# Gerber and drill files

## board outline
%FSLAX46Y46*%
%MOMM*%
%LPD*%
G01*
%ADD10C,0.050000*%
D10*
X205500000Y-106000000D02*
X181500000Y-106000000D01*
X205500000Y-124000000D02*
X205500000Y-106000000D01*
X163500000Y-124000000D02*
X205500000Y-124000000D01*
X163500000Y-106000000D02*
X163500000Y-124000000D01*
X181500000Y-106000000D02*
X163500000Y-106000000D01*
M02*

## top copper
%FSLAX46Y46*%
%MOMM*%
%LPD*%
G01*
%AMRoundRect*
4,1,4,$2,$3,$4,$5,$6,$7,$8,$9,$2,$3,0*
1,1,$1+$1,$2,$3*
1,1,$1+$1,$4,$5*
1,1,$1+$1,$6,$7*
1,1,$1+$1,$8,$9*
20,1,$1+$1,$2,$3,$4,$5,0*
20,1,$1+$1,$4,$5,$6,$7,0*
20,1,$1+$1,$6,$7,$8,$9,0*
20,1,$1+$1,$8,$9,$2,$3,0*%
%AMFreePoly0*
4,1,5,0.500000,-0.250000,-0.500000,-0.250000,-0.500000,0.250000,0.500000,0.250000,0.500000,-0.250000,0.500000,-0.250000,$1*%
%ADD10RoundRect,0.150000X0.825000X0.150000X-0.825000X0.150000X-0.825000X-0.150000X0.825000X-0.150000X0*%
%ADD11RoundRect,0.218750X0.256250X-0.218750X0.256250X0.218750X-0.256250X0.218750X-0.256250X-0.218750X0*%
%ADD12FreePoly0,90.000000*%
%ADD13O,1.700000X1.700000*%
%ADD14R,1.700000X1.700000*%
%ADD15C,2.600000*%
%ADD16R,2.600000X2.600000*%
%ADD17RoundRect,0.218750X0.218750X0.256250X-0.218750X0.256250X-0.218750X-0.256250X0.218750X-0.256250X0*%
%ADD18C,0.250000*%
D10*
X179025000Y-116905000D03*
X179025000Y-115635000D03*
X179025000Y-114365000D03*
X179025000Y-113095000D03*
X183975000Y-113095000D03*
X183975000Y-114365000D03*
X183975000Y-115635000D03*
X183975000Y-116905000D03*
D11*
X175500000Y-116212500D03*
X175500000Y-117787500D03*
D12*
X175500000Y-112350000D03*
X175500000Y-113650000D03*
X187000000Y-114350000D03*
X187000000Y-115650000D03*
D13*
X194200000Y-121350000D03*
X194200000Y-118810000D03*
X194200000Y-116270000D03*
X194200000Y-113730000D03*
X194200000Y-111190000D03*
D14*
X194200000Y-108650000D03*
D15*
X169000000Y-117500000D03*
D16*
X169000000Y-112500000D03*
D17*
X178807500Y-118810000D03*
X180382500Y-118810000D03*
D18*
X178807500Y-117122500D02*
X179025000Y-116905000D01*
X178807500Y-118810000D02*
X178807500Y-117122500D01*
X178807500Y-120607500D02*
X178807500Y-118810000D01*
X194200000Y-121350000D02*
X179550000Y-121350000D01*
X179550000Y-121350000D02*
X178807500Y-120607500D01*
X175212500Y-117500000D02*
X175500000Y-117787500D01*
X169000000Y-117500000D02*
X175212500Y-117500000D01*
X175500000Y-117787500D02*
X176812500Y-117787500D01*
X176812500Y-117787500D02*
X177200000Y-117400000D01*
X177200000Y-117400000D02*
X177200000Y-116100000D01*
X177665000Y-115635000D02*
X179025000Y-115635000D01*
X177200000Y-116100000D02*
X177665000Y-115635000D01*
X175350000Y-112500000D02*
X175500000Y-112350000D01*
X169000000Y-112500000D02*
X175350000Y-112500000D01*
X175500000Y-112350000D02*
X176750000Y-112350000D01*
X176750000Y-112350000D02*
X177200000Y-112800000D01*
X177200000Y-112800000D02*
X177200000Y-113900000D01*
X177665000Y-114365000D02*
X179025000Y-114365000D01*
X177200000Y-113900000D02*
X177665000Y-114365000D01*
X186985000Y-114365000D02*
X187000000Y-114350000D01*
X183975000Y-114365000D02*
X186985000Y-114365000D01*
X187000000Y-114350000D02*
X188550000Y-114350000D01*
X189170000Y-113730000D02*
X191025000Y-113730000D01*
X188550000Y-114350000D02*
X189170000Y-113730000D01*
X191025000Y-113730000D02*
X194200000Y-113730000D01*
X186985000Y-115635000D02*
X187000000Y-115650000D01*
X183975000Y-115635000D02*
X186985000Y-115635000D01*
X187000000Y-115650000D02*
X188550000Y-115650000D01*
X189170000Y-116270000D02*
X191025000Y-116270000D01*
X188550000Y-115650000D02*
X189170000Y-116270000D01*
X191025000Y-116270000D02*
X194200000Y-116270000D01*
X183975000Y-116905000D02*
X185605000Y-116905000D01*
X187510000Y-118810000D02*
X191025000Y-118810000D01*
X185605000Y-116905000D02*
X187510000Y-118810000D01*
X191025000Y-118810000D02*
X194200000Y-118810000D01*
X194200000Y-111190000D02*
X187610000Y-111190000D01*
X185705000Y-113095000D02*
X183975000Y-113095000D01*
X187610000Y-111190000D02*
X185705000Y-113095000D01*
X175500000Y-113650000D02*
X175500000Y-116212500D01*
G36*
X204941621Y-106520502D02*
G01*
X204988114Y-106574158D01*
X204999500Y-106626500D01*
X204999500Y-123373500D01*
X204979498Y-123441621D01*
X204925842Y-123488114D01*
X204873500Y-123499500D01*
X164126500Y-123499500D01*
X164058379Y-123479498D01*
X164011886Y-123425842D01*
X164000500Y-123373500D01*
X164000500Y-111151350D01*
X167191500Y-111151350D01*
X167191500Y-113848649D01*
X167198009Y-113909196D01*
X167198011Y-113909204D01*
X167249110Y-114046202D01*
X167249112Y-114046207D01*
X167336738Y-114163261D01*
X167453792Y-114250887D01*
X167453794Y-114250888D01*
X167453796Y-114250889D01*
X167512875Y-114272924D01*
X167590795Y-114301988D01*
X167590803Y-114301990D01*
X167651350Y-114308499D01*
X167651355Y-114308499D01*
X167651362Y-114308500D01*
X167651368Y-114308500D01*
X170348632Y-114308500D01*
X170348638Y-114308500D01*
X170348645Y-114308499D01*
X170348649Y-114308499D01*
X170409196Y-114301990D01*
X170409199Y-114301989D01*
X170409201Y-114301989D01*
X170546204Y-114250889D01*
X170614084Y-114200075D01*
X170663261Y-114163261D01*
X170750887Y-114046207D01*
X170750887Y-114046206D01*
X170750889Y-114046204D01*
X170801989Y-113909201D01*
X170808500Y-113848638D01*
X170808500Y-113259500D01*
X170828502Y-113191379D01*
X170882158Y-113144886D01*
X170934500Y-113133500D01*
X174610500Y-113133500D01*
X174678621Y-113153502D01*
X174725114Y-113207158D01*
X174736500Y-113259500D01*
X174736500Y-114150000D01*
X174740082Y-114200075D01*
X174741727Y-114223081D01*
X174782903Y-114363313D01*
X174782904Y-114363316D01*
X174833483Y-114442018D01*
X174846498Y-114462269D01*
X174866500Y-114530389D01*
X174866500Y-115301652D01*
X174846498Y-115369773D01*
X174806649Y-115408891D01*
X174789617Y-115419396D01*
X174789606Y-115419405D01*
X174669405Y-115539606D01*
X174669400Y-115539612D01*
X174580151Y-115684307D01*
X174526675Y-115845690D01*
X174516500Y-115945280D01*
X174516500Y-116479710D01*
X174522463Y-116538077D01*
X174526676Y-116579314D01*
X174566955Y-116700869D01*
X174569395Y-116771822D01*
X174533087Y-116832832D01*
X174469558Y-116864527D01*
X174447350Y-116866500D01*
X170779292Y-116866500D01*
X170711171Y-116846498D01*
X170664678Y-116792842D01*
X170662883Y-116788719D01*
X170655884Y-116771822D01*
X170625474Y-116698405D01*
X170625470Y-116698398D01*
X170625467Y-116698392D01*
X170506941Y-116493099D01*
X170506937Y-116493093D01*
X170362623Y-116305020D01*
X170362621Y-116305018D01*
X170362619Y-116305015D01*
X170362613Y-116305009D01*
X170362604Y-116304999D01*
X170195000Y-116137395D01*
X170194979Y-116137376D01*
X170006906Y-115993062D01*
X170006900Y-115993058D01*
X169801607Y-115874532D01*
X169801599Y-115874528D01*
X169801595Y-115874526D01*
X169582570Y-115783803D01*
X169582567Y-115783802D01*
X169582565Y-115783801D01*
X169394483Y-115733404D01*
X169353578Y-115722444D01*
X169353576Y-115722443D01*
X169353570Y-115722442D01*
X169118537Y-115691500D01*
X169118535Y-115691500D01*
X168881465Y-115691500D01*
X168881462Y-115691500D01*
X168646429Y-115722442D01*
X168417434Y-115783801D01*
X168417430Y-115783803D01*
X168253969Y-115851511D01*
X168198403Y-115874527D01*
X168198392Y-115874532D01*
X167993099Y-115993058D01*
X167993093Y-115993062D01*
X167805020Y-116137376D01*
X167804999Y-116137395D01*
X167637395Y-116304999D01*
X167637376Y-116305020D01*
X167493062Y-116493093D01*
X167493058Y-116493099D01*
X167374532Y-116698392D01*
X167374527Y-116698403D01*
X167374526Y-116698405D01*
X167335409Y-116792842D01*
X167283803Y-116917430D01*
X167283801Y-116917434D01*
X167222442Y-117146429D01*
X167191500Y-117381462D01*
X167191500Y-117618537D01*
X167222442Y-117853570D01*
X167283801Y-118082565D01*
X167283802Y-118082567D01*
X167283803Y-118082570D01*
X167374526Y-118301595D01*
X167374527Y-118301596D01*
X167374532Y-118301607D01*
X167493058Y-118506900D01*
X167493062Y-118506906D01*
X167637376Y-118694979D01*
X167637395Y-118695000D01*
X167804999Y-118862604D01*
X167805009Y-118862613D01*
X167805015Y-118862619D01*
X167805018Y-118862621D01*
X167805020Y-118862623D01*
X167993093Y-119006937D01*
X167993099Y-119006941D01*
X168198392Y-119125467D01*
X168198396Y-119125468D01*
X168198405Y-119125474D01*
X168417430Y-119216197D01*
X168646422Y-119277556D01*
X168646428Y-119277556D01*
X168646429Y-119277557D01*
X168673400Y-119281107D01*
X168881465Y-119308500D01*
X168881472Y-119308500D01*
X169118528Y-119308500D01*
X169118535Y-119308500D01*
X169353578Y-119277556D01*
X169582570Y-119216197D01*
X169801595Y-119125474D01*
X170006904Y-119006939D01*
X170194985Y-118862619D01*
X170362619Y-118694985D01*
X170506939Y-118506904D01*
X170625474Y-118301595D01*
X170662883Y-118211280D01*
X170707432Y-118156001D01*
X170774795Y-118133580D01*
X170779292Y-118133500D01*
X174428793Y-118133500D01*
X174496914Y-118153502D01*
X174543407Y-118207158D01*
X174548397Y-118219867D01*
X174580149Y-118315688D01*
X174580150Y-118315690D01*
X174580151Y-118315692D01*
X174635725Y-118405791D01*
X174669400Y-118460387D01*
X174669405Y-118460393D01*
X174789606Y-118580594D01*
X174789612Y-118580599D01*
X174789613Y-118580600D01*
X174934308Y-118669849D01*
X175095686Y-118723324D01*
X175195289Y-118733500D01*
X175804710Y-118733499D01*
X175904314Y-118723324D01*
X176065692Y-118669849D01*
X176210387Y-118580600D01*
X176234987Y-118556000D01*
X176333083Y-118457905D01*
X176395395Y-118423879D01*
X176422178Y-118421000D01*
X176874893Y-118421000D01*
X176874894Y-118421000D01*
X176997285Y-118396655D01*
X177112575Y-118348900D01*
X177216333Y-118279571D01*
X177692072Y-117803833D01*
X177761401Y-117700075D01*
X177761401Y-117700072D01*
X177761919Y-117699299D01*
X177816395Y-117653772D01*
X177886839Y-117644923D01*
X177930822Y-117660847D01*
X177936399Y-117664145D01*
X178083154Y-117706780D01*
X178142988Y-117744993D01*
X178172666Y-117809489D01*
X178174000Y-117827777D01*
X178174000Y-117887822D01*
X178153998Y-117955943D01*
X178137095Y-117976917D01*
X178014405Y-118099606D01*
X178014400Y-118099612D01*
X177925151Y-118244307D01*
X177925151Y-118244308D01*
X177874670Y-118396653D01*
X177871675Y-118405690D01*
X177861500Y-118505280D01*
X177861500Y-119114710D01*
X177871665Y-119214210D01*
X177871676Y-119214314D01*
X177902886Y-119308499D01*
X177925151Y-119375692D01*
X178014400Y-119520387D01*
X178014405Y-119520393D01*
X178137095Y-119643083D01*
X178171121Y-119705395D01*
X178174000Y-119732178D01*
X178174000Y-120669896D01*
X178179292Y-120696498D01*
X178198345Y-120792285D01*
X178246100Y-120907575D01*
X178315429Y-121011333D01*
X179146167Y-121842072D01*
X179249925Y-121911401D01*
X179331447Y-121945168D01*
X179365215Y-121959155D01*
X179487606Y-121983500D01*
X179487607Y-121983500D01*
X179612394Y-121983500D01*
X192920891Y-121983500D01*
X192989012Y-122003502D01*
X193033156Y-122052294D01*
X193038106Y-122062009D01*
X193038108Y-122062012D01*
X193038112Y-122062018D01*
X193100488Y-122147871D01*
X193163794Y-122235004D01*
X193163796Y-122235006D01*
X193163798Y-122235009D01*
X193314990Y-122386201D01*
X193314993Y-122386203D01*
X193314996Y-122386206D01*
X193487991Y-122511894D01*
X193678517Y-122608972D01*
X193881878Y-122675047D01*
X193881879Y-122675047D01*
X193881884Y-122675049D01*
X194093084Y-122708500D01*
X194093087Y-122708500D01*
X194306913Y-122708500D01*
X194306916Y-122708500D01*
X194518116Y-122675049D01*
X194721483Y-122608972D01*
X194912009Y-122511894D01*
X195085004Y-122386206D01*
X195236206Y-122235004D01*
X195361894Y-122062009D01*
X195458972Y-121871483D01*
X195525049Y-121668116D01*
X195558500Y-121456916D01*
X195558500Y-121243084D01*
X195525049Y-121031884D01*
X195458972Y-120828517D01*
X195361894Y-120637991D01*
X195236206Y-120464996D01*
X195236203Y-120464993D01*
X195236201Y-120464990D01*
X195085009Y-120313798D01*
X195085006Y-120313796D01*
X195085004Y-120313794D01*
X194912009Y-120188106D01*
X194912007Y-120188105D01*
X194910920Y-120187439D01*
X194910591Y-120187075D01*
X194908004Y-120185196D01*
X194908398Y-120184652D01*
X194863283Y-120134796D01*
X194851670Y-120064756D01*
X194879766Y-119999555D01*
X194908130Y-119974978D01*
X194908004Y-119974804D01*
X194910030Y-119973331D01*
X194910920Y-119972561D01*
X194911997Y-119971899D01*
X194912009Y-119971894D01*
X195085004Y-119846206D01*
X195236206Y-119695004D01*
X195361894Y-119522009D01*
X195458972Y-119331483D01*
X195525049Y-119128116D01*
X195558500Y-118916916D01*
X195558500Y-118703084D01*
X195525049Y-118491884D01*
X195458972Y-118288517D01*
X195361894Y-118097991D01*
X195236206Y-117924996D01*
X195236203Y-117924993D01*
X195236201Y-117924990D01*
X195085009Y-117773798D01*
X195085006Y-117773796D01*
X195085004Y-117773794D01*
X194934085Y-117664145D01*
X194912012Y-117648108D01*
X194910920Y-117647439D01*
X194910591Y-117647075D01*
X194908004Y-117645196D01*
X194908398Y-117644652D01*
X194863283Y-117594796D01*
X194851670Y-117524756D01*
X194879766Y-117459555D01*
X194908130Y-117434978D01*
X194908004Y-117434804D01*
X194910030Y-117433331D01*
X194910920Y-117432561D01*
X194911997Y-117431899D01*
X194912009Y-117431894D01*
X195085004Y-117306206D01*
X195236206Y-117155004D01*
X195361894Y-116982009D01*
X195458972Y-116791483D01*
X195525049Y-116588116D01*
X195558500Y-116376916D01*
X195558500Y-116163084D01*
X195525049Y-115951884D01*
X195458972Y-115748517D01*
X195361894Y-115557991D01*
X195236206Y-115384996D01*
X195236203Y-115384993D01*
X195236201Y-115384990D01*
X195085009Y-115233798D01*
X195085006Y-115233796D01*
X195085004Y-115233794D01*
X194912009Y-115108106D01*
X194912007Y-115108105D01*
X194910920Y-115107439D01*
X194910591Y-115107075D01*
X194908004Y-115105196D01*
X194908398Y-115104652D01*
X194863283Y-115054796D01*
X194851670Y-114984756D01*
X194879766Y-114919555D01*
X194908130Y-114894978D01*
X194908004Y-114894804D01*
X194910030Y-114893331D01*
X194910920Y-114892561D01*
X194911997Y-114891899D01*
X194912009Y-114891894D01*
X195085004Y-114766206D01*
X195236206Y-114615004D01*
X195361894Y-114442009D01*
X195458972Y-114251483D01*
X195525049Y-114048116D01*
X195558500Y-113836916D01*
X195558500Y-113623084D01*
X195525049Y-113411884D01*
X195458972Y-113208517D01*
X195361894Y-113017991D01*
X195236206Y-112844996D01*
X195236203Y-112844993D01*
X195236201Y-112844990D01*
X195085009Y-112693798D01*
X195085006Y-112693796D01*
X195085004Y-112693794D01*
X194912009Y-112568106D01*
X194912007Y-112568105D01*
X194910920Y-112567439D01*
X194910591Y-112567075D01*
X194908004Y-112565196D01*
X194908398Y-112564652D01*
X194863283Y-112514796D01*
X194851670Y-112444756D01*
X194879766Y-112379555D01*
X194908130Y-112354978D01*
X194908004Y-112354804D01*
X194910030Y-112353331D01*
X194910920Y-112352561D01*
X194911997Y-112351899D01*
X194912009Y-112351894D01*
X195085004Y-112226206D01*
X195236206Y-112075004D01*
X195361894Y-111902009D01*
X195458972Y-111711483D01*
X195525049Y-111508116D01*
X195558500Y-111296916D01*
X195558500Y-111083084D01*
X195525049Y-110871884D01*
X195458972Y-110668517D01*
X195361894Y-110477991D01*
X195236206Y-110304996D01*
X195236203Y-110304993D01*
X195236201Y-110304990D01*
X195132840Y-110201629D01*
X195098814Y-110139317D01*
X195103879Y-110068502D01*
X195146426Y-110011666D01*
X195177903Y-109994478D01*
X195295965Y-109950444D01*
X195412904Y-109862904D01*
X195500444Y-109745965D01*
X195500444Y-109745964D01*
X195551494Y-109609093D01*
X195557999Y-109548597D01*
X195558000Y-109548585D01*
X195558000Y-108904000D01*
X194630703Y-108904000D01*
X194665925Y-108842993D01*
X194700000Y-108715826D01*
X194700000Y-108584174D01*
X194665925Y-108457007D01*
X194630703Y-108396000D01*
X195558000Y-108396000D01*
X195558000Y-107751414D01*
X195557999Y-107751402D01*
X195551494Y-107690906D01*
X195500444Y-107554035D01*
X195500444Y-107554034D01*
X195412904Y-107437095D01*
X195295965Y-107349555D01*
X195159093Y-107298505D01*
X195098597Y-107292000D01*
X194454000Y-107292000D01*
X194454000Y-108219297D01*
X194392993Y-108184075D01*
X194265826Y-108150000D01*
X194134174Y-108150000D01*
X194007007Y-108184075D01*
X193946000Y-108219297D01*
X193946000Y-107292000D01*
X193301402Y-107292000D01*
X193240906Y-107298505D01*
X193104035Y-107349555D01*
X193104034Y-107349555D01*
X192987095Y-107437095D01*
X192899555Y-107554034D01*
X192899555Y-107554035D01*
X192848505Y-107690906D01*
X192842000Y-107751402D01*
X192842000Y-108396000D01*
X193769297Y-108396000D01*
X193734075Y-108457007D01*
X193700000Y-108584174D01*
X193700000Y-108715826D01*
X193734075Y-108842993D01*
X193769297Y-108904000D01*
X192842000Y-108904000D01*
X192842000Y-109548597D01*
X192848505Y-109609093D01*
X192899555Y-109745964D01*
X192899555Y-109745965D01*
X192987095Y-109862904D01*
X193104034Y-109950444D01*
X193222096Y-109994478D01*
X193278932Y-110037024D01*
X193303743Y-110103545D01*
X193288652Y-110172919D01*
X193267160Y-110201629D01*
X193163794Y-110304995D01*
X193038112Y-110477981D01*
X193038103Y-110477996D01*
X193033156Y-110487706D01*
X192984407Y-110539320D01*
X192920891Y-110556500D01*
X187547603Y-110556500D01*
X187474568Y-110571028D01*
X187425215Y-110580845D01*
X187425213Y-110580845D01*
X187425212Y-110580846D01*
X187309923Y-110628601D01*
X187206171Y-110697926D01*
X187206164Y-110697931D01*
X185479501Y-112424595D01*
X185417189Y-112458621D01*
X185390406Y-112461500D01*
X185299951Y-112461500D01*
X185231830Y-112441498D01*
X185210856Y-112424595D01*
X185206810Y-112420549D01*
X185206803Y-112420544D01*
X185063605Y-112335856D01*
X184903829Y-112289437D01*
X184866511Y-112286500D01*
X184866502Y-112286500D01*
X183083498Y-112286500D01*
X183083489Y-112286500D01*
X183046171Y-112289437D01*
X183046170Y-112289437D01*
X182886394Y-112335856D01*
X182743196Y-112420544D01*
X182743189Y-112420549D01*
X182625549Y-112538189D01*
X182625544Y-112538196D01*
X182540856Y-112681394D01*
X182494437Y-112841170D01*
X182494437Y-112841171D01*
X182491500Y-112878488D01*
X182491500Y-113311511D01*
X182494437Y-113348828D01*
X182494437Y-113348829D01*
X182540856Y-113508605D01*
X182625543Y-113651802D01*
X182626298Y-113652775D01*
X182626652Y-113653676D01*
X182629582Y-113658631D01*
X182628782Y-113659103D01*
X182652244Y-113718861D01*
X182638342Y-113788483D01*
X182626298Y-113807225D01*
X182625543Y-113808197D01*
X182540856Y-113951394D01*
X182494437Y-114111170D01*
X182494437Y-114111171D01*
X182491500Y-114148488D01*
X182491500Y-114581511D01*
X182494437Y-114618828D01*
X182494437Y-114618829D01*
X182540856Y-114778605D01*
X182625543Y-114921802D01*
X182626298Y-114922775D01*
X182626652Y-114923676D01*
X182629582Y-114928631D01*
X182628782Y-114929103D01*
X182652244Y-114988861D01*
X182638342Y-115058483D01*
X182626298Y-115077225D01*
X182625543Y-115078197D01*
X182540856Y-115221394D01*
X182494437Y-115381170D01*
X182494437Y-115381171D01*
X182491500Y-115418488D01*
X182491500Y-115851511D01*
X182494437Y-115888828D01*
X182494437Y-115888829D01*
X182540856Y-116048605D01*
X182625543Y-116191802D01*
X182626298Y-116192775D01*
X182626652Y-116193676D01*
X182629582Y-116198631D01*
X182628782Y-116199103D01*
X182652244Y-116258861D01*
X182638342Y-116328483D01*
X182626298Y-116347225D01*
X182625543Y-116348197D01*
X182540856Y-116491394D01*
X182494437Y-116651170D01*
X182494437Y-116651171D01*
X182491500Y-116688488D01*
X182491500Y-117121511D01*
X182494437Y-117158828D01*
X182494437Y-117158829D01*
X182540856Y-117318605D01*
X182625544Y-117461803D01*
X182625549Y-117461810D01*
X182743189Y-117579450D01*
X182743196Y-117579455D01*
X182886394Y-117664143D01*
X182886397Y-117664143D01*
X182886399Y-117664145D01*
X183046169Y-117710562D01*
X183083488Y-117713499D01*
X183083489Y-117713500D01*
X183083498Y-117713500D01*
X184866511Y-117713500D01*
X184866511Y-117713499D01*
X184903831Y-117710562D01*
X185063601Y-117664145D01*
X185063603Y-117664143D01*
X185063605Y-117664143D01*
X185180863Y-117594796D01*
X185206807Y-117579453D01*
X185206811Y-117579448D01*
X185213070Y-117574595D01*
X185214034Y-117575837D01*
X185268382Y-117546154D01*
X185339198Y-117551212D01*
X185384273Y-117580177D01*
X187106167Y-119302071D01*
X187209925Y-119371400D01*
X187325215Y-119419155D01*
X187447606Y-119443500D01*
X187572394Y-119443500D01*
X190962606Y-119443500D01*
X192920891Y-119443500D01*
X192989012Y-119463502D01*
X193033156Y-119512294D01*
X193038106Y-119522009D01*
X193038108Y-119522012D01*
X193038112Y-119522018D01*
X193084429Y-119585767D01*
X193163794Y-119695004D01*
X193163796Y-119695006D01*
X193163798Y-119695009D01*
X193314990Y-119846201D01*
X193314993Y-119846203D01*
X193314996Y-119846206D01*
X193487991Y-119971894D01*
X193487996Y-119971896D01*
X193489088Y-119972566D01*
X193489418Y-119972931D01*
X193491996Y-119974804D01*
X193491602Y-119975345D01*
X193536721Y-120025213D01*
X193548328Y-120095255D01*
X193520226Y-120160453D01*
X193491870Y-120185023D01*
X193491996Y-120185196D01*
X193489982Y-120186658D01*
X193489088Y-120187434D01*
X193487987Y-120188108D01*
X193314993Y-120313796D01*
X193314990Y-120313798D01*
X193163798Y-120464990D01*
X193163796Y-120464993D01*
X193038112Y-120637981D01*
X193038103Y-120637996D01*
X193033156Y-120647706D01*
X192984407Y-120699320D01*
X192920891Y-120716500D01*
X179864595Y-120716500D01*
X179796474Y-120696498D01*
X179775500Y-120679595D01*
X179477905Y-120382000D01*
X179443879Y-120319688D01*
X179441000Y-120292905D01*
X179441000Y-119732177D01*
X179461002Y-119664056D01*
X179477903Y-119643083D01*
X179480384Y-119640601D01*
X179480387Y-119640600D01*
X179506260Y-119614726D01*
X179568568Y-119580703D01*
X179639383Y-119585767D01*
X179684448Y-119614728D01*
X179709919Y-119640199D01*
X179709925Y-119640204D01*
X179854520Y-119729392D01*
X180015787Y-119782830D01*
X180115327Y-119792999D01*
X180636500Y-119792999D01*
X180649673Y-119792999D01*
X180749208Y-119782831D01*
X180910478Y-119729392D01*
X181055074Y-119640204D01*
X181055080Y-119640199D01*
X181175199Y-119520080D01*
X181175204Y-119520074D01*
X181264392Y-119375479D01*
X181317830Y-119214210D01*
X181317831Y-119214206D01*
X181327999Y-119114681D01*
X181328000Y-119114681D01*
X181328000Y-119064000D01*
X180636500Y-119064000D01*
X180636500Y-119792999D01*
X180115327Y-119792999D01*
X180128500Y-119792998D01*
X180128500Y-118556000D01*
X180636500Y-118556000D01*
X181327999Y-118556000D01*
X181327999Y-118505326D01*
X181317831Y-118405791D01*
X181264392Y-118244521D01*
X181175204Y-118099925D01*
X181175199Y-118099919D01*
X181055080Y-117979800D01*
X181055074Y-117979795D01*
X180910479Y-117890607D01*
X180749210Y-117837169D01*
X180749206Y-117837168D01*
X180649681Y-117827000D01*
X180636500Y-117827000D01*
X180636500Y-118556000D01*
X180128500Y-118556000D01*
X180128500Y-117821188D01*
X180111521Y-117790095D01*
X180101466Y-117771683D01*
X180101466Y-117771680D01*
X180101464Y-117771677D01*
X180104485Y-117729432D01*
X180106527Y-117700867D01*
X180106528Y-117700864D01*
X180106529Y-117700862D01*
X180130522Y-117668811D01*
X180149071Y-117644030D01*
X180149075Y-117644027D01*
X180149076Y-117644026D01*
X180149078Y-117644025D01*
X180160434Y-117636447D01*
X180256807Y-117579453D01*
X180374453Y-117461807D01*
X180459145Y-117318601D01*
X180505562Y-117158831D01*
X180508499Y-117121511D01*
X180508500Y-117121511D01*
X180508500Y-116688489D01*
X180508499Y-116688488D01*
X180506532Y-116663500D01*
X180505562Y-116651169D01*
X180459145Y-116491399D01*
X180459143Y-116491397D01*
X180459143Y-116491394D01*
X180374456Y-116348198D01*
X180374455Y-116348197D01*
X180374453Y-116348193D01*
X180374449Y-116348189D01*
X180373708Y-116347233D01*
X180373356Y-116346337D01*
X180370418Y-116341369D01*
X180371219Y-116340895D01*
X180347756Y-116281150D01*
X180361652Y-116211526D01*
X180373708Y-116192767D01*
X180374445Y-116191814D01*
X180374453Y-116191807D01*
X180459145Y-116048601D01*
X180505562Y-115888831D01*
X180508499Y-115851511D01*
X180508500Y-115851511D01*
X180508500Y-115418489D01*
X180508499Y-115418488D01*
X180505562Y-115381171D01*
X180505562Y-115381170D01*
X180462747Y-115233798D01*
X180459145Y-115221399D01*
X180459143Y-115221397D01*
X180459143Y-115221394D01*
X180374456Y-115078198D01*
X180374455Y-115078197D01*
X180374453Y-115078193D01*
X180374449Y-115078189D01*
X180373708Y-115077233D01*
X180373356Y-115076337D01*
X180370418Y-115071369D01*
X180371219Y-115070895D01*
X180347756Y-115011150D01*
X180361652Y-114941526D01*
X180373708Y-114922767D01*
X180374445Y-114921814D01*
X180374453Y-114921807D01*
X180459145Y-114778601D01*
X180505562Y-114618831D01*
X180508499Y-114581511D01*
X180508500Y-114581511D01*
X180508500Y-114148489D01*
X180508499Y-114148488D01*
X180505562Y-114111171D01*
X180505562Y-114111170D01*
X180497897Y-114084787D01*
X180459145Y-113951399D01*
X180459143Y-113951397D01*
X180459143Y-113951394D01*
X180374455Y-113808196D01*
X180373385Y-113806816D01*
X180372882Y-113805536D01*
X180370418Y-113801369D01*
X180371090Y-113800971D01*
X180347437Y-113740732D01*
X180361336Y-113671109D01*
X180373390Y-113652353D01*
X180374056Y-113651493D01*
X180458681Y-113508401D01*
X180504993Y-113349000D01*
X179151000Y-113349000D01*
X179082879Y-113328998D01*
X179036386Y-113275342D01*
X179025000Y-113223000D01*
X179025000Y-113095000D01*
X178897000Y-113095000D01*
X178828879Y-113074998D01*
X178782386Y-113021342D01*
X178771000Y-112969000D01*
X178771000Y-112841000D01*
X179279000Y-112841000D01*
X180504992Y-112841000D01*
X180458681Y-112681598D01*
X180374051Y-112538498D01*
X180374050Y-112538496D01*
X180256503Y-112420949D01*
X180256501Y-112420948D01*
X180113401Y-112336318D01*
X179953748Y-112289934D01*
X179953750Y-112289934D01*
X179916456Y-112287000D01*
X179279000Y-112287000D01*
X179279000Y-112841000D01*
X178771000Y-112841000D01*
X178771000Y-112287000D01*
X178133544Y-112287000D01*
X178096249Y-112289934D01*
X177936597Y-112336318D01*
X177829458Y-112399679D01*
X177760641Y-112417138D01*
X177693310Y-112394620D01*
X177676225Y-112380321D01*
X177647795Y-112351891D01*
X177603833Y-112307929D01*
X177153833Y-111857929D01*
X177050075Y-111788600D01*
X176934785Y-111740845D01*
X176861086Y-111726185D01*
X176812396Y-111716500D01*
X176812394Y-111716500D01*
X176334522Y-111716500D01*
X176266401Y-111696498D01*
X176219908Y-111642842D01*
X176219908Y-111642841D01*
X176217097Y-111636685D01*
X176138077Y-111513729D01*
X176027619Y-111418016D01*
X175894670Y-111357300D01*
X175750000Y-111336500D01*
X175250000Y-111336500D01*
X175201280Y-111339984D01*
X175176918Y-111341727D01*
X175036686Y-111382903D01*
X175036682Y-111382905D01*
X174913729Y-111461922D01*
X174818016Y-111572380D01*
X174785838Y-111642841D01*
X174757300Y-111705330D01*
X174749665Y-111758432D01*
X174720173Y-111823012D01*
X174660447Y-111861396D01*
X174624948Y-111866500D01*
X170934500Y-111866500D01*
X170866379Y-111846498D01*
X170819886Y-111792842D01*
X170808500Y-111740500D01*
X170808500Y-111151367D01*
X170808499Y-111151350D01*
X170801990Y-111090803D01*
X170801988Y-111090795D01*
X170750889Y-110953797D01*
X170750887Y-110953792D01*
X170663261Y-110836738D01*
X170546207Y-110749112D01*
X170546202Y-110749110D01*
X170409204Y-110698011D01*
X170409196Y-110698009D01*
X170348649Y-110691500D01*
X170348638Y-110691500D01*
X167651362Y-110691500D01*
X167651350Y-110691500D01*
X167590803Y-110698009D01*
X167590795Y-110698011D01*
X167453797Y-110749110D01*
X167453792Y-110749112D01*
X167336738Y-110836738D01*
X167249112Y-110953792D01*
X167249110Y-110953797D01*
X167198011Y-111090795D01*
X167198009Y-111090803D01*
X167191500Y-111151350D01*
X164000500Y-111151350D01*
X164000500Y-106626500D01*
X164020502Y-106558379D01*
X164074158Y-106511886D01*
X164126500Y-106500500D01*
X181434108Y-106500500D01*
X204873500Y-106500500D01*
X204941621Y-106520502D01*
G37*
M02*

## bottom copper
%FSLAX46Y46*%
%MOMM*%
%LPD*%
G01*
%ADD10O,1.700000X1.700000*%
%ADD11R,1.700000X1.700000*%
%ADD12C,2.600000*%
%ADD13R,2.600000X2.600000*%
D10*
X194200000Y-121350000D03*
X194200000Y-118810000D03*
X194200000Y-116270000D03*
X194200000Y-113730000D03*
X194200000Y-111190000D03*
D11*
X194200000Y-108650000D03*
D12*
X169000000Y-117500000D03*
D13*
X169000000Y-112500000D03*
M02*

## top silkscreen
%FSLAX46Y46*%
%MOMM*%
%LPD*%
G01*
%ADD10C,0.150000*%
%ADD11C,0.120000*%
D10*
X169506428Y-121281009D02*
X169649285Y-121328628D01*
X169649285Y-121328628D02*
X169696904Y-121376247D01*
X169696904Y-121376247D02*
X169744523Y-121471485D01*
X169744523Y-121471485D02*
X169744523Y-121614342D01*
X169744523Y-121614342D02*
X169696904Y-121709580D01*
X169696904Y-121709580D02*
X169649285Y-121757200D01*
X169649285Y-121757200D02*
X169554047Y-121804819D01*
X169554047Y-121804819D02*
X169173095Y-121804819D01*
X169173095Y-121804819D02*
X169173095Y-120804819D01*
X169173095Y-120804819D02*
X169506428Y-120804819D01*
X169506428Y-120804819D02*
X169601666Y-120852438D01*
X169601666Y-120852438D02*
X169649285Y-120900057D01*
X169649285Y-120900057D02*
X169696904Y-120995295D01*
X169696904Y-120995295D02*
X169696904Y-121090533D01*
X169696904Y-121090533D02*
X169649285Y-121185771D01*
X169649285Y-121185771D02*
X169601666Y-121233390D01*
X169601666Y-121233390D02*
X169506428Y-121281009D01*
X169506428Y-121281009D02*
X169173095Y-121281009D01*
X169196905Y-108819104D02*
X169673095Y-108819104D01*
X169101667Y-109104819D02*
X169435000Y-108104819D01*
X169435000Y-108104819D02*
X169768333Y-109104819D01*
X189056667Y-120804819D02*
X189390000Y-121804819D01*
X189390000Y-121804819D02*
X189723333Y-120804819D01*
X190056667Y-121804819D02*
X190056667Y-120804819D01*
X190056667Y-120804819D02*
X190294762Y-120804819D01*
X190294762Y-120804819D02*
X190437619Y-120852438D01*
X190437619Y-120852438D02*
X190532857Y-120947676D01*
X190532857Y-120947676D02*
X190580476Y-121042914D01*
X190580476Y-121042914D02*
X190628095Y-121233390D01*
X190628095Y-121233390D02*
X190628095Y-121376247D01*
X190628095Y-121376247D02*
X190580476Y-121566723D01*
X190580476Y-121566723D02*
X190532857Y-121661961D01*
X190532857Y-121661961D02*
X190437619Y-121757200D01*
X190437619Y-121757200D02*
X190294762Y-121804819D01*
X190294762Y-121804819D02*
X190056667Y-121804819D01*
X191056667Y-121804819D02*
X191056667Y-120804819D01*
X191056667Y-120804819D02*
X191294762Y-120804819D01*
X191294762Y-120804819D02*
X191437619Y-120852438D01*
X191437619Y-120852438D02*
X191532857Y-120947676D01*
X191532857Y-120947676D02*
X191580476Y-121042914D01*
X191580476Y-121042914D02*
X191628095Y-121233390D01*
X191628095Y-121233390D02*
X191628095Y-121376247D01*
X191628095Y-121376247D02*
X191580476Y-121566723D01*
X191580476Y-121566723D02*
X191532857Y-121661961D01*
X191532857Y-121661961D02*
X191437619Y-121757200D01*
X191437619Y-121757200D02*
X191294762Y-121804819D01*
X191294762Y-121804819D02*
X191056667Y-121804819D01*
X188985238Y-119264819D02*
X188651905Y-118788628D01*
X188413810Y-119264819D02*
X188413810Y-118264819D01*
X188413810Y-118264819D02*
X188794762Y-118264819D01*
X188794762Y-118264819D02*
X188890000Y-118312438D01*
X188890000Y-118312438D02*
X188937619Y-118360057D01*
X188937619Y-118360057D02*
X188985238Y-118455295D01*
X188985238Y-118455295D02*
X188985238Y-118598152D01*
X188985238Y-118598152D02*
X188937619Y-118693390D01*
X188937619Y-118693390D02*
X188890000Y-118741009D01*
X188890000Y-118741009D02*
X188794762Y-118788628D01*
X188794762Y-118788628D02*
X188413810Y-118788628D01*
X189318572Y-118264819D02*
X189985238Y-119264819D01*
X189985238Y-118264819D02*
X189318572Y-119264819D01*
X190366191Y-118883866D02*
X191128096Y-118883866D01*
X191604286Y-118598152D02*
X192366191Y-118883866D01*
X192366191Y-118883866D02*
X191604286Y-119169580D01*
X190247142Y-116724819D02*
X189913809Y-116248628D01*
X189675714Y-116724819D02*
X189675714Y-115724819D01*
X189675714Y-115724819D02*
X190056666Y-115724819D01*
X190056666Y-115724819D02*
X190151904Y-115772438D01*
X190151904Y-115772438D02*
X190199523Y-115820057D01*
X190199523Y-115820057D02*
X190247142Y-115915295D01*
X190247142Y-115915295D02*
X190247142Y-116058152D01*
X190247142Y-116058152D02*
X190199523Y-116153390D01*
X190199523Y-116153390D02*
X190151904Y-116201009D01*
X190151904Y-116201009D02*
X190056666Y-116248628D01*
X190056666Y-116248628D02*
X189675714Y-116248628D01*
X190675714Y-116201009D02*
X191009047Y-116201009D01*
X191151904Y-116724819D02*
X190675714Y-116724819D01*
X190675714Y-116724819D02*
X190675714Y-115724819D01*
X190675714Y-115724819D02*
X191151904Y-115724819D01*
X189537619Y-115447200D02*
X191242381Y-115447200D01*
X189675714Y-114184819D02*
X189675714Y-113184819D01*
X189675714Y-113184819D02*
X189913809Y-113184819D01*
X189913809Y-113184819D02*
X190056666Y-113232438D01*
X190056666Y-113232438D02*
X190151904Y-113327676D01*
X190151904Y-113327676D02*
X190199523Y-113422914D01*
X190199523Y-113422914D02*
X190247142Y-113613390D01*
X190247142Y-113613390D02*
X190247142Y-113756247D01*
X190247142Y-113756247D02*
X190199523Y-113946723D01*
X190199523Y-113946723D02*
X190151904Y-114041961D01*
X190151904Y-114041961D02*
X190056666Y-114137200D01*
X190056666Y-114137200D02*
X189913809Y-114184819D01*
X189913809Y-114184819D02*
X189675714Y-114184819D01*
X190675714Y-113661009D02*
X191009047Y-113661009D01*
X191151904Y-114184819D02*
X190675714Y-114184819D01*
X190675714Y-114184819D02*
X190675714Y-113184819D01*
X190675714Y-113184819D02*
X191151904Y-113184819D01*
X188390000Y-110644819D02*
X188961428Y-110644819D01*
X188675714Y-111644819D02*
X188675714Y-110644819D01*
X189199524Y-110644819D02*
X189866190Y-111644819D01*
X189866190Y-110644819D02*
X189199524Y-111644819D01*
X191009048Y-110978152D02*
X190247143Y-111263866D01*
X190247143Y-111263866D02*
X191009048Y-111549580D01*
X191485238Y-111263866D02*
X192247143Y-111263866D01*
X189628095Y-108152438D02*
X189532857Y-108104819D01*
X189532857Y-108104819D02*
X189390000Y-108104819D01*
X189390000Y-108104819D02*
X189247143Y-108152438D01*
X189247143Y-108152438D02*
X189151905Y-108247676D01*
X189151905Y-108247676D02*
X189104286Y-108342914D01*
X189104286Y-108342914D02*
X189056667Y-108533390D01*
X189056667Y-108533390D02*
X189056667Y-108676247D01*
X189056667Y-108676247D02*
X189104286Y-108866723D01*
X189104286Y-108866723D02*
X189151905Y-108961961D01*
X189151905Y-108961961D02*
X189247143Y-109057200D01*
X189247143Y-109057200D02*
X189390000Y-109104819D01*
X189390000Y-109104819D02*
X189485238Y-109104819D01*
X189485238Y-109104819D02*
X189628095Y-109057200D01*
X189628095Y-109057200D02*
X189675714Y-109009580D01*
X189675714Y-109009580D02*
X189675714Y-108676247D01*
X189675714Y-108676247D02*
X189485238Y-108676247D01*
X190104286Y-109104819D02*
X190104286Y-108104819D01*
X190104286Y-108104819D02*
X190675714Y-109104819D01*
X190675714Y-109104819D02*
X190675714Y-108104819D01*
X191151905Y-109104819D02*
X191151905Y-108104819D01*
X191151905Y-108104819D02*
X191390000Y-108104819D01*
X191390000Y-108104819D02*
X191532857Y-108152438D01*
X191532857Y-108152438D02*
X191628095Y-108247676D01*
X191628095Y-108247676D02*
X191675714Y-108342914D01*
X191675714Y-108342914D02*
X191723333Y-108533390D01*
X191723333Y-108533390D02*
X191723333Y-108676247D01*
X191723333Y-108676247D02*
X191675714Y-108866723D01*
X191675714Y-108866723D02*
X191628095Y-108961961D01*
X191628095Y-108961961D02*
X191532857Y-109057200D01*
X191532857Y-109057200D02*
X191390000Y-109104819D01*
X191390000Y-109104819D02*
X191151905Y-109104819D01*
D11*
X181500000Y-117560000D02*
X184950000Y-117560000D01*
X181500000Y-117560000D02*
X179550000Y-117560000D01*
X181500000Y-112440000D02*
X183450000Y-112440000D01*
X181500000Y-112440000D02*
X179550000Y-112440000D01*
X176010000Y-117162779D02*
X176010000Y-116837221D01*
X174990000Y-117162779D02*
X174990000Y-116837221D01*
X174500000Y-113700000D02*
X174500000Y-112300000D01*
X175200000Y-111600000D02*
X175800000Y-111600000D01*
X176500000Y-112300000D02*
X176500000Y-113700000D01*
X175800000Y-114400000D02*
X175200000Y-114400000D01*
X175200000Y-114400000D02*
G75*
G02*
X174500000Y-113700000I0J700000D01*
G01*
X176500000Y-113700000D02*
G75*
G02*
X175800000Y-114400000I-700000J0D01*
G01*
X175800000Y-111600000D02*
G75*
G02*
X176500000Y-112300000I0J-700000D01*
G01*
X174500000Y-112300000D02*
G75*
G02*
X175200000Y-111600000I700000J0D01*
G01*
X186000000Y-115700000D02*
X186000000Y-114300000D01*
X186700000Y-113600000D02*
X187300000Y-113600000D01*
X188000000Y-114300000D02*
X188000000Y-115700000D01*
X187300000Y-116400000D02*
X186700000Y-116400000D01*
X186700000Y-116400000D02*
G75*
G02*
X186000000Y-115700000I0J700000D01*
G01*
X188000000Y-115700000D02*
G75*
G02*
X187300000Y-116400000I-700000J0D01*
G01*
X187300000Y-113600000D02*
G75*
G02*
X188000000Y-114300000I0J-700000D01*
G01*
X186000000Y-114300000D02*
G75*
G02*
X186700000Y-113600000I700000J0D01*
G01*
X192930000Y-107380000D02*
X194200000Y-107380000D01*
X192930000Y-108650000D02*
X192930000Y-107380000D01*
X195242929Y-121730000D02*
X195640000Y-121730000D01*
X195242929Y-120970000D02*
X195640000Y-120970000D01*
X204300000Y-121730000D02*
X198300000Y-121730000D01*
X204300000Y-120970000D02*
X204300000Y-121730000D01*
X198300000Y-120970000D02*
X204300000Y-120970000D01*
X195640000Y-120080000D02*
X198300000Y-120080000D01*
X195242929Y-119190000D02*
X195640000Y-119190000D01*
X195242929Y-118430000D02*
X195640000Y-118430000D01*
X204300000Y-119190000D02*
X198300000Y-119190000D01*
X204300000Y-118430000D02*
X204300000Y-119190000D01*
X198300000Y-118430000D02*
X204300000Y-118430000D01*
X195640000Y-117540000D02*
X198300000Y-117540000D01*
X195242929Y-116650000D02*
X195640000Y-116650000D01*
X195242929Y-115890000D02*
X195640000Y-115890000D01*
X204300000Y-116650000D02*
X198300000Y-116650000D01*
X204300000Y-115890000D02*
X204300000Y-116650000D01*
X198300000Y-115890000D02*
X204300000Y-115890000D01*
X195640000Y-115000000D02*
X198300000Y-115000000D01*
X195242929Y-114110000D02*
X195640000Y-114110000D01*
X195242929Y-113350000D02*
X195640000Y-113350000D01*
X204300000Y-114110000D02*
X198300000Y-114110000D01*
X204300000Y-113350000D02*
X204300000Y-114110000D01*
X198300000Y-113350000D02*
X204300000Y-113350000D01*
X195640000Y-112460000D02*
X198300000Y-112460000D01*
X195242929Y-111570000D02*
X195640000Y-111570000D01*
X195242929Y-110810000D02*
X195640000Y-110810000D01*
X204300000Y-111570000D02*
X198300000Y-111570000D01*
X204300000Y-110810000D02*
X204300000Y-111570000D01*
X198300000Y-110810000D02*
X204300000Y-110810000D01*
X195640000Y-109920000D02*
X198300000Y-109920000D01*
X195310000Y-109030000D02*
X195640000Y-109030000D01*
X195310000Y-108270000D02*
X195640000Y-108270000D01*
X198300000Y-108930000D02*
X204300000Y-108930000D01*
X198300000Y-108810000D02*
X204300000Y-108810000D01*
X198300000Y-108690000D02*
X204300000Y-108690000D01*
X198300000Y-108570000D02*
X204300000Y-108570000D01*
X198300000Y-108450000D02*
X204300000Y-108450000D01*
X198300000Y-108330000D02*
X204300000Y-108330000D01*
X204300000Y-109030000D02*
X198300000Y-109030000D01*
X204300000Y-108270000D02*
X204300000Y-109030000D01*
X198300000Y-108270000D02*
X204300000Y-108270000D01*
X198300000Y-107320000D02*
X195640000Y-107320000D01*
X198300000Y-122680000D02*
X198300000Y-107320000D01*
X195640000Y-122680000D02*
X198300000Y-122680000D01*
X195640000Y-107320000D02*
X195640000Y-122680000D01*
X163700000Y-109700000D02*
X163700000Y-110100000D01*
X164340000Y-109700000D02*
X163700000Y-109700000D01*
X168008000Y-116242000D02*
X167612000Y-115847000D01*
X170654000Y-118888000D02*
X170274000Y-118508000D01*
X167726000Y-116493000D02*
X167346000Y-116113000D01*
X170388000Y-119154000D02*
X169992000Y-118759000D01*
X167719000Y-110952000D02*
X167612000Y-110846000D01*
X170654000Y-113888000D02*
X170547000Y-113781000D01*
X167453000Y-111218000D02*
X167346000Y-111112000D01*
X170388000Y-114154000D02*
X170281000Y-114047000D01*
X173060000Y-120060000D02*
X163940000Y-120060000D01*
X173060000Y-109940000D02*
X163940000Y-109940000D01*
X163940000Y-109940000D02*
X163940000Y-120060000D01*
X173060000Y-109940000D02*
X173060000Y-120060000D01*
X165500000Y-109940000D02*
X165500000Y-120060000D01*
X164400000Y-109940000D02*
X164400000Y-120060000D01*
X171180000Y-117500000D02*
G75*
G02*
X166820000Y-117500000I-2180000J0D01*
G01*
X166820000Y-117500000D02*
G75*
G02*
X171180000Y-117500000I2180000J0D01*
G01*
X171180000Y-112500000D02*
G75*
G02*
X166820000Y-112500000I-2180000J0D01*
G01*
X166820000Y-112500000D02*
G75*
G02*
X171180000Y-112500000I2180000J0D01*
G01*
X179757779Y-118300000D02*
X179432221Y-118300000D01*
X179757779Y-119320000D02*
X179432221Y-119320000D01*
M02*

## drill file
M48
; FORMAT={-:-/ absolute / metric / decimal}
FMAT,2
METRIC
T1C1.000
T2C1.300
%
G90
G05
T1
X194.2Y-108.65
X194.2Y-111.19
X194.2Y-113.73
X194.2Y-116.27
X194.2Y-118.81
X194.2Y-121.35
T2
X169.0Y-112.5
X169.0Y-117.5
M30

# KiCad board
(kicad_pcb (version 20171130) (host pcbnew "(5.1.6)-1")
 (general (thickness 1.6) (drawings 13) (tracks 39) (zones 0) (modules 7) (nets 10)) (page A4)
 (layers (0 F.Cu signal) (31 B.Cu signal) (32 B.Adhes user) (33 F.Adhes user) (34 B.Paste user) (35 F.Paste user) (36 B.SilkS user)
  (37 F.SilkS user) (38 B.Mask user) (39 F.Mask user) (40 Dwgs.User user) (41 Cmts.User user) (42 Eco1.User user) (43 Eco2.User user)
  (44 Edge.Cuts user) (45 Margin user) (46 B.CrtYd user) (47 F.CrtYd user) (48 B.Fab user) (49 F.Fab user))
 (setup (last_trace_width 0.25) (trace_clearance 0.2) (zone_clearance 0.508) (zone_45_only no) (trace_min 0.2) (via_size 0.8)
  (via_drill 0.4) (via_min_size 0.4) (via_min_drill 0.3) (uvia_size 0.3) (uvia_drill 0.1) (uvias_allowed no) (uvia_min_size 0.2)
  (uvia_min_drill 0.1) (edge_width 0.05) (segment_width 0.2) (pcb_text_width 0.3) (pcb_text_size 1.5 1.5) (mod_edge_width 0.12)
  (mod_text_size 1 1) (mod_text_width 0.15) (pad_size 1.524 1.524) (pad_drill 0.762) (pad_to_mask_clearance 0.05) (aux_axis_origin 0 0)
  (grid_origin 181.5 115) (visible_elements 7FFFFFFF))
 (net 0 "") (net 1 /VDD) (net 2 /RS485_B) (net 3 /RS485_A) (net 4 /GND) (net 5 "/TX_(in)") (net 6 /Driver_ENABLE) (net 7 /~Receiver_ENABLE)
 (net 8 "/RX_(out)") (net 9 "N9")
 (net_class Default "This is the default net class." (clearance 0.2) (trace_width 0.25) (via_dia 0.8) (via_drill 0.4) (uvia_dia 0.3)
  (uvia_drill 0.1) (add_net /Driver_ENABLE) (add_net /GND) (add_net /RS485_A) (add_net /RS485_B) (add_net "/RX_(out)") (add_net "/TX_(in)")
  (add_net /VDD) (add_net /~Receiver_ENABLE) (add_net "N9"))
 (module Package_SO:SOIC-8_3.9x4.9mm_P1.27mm (layer F.Cu) (at 181.5 115 180)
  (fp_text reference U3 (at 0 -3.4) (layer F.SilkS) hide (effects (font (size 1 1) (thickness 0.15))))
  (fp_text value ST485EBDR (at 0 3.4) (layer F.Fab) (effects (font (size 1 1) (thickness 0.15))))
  (fp_line (start 0 -2.56) (end -3.45 -2.56) (layer F.SilkS) (width 0.12))
  (fp_line (start 0 -2.56) (end 1.95 -2.56) (layer F.SilkS) (width 0.12))
  (fp_line (start 0 2.56) (end -1.95 2.56) (layer F.SilkS) (width 0.12))
  (fp_line (start 0 2.56) (end 1.95 2.56) (layer F.SilkS) (width 0.12))
  (pad 8 smd roundrect (at 2.475 -1.905 180) (size 1.95 0.6) (layers F.Cu F.Paste F.Mask) (roundrect_rratio 0.25) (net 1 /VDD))
  (pad 7 smd roundrect (at 2.475 -0.635 180) (size 1.95 0.6) (layers F.Cu F.Paste F.Mask) (roundrect_rratio 0.25) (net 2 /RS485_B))
  (pad 6 smd roundrect (at 2.475 0.635 180) (size 1.95 0.6) (layers F.Cu F.Paste F.Mask) (roundrect_rratio 0.25) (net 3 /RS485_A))
  (pad 5 smd roundrect (at 2.475 1.905 180) (size 1.95 0.6) (layers F.Cu F.Paste F.Mask) (roundrect_rratio 0.25) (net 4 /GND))
  (pad 4 smd roundrect (at -2.475 1.905 180) (size 1.95 0.6) (layers F.Cu F.Paste F.Mask) (roundrect_rratio 0.25) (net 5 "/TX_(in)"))
  (pad 3 smd roundrect (at -2.475 0.635 180) (size 1.95 0.6) (layers F.Cu F.Paste F.Mask) (roundrect_rratio 0.25) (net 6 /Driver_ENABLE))
  (pad 2 smd roundrect (at -2.475 -0.635 180) (size 1.95 0.6) (layers F.Cu F.Paste F.Mask) (roundrect_rratio 0.25) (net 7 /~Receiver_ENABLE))
  (pad 1 smd roundrect (at -2.475 -1.905 180) (size 1.95 0.6) (layers F.Cu F.Paste F.Mask) (roundrect_rratio 0.25) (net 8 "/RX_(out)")))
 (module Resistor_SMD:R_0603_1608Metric (layer F.Cu) (at 175.5 117 90)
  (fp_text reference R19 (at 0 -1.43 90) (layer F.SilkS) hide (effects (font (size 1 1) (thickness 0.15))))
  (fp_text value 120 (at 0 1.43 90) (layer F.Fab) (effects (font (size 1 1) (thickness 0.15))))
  (fp_line (start -0.162779 0.51) (end 0.162779 0.51) (layer F.SilkS) (width 0.12))
  (fp_line (start -0.162779 -0.51) (end 0.162779 -0.51) (layer F.SilkS) (width 0.12))
  (pad 2 smd roundrect (at 0.7875 0 90) (size 0.875 0.95) (layers F.Cu F.Paste F.Mask) (roundrect_rratio 0.25) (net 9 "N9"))
  (pad 1 smd roundrect (at -0.7875 0 90) (size 0.875 0.95) (layers F.Cu F.Paste F.Mask) (roundrect_rratio 0.25) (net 2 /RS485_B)))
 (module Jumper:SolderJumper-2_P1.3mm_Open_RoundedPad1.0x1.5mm (layer F.Cu) (at 175.5 113 90)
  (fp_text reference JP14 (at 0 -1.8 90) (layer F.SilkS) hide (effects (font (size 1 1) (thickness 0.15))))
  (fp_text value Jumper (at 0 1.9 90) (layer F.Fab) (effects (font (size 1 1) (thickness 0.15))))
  (fp_line (start -0.7 -1) (end 0.7 -1) (layer F.SilkS) (width 0.12))
  (fp_line (start 1.4 -0.3) (end 1.4 0.3) (layer F.SilkS) (width 0.12))
  (fp_line (start 0.7 1) (end -0.7 1) (layer F.SilkS) (width 0.12))
  (fp_line (start -1.4 0.3) (end -1.4 -0.3) (layer F.SilkS) (width 0.12))
  (fp_arc (start -0.7 -0.3) (end -0.7 -1) (angle -90) (layer F.SilkS) (width 0.12))
  (fp_arc (start -0.7 0.3) (end -1.4 0.3) (angle -90) (layer F.SilkS) (width 0.12))
  (fp_arc (start 0.7 0.3) (end 0.7 1) (angle -90) (layer F.SilkS) (width 0.12))
  (fp_arc (start 0.7 -0.3) (end 1.4 -0.3) (angle -90) (layer F.SilkS) (width 0.12))
  (pad 2 smd custom (at 0.65 0 90) (size 1 0.5) (layers F.Cu F.Mask) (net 3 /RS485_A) (zone_connect 2)
   (options (clearance outline) (anchor rect)) (primitives))
  (pad 1 smd custom (at -0.65 0 90) (size 1 0.5) (layers F.Cu F.Mask) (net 9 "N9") (zone_connect 2)
   (options (clearance outline) (anchor rect)) (primitives)))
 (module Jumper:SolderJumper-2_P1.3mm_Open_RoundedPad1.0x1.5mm (layer F.Cu) (at 187 115 90)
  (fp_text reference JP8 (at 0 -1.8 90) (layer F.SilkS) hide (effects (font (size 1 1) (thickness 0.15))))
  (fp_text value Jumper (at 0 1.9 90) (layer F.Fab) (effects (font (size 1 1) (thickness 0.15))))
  (fp_line (start -0.7 -1) (end 0.7 -1) (layer F.SilkS) (width 0.12))
  (fp_line (start 1.4 -0.3) (end 1.4 0.3) (layer F.SilkS) (width 0.12))
  (fp_line (start 0.7 1) (end -0.7 1) (layer F.SilkS) (width 0.12))
  (fp_line (start -1.4 0.3) (end -1.4 -0.3) (layer F.SilkS) (width 0.12))
  (fp_arc (start -0.7 -0.3) (end -0.7 -1) (angle -90) (layer F.SilkS) (width 0.12))
  (fp_arc (start -0.7 0.3) (end -1.4 0.3) (angle -90) (layer F.SilkS) (width 0.12))
  (fp_arc (start 0.7 0.3) (end 0.7 1) (angle -90) (layer F.SilkS) (width 0.12))
  (fp_arc (start 0.7 -0.3) (end 1.4 -0.3) (angle -90) (layer F.SilkS) (width 0.12))
  (pad 2 smd custom (at 0.65 0 90) (size 1 0.5) (layers F.Cu F.Mask) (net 6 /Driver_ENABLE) (zone_connect 2)
   (options (clearance outline) (anchor rect)) (primitives))
  (pad 1 smd custom (at -0.65 0 90) (size 1 0.5) (layers F.Cu F.Mask) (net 7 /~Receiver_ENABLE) (zone_connect 2)
   (options (clearance outline) (anchor rect)) (primitives)))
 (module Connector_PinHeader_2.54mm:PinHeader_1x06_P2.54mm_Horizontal (layer F.Cu) (at 194.2 108.65)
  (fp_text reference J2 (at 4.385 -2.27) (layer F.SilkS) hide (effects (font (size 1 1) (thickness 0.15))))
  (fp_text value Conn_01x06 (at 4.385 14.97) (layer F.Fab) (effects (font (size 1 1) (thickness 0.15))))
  (fp_line (start -1.27 -1.27) (end 0 -1.27) (layer F.SilkS) (width 0.12))
  (fp_line (start -1.27 0) (end -1.27 -1.27) (layer F.SilkS) (width 0.12))
  (fp_line (start 1.042929 13.08) (end 1.44 13.08) (layer F.SilkS) (width 0.12))
  (fp_line (start 1.042929 12.32) (end 1.44 12.32) (layer F.SilkS) (width 0.12))
  (fp_line (start 10.1 13.08) (end 4.1 13.08) (layer F.SilkS) (width 0.12))
  (fp_line (start 10.1 12.32) (end 10.1 13.08) (layer F.SilkS) (width 0.12))
  (fp_line (start 4.1 12.32) (end 10.1 12.32) (layer F.SilkS) (width 0.12))
  (fp_line (start 1.44 11.43) (end 4.1 11.43) (layer F.SilkS) (width 0.12))
  (fp_line (start 1.042929 10.54) (end 1.44 10.54) (layer F.SilkS) (width 0.12))
  (fp_line (start 1.042929 9.78) (end 1.44 9.78) (layer F.SilkS) (width 0.12))
  (fp_line (start 10.1 10.54) (end 4.1 10.54) (layer F.SilkS) (width 0.12))
  (fp_line (start 10.1 9.78) (end 10.1 10.54) (layer F.SilkS) (width 0.12))
  (fp_line (start 4.1 9.78) (end 10.1 9.78) (layer F.SilkS) (width 0.12))
  (fp_line (start 1.44 8.89) (end 4.1 8.89) (layer F.SilkS) (width 0.12))
  (fp_line (start 1.042929 8) (end 1.44 8) (layer F.SilkS) (width 0.12))
  (fp_line (start 1.042929 7.24) (end 1.44 7.24) (layer F.SilkS) (width 0.12))
  (fp_line (start 10.1 8) (end 4.1 8) (layer F.SilkS) (width 0.12))
  (fp_line (start 10.1 7.24) (end 10.1 8) (layer F.SilkS) (width 0.12))
  (fp_line (start 4.1 7.24) (end 10.1 7.24) (layer F.SilkS) (width 0.12))
  (fp_line (start 1.44 6.35) (end 4.1 6.35) (layer F.SilkS) (width 0.12))
  (fp_line (start 1.042929 5.46) (end 1.44 5.46) (layer F.SilkS) (width 0.12))
  (fp_line (start 1.042929 4.7) (end 1.44 4.7) (layer F.SilkS) (width 0.12))
  (fp_line (start 10.1 5.46) (end 4.1 5.46) (layer F.SilkS) (width 0.12))
  (fp_line (start 10.1 4.7) (end 10.1 5.46) (layer F.SilkS) (width 0.12))
  (fp_line (start 4.1 4.7) (end 10.1 4.7) (layer F.SilkS) (width 0.12))
  (fp_line (start 1.44 3.81) (end 4.1 3.81) (layer F.SilkS) (width 0.12))
  (fp_line (start 1.042929 2.92) (end 1.44 2.92) (layer F.SilkS) (width 0.12))
  (fp_line (start 1.042929 2.16) (end 1.44 2.16) (layer F.SilkS) (width 0.12))
  (fp_line (start 10.1 2.92) (end 4.1 2.92) (layer F.SilkS) (width 0.12))
  (fp_line (start 10.1 2.16) (end 10.1 2.92) (layer F.SilkS) (width 0.12))
  (fp_line (start 4.1 2.16) (end 10.1 2.16) (layer F.SilkS) (width 0.12))
  (fp_line (start 1.44 1.27) (end 4.1 1.27) (layer F.SilkS) (width 0.12))
  (fp_line (start 1.11 0.38) (end 1.44 0.38) (layer F.SilkS) (width 0.12))
  (fp_line (start 1.11 -0.38) (end 1.44 -0.38) (layer F.SilkS) (width 0.12))
  (fp_line (start 4.1 0.28) (end 10.1 0.28) (layer F.SilkS) (width 0.12))
  (fp_line (start 4.1 0.16) (end 10.1 0.16) (layer F.SilkS) (width 0.12))
  (fp_line (start 4.1 0.04) (end 10.1 0.04) (layer F.SilkS) (width 0.12))
  (fp_line (start 4.1 -0.08) (end 10.1 -0.08) (layer F.SilkS) (width 0.12))
  (fp_line (start 4.1 -0.2) (end 10.1 -0.2) (layer F.SilkS) (width 0.12))
  (fp_line (start 4.1 -0.32) (end 10.1 -0.32) (layer F.SilkS) (width 0.12))
  (fp_line (start 10.1 0.38) (end 4.1 0.38) (layer F.SilkS) (width 0.12))
  (fp_line (start 10.1 -0.38) (end 10.1 0.38) (layer F.SilkS) (width 0.12))
  (fp_line (start 4.1 -0.38) (end 10.1 -0.38) (layer F.SilkS) (width 0.12))
  (fp_line (start 4.1 -1.33) (end 1.44 -1.33) (layer F.SilkS) (width 0.12))
  (fp_line (start 4.1 14.03) (end 4.1 -1.33) (layer F.SilkS) (width 0.12))
  (fp_line (start 1.44 14.03) (end 4.1 14.03) (layer F.SilkS) (width 0.12))
  (fp_line (start 1.44 -1.33) (end 1.44 14.03) (layer F.SilkS) (width 0.12))
  (pad 6 thru_hole oval (at 0 12.7) (size 1.7 1.7) (drill 1) (layers *.Cu *.Mask) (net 1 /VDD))
  (pad 5 thru_hole oval (at 0 10.16) (size 1.7 1.7) (drill 1) (layers *.Cu *.Mask) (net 8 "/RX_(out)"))
  (pad 4 thru_hole oval (at 0 7.62) (size 1.7 1.7) (drill 1) (layers *.Cu *.Mask) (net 7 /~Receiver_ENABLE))
  (pad 3 thru_hole oval (at 0 5.08) (size 1.7 1.7) (drill 1) (layers *.Cu *.Mask) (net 6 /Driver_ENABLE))
  (pad 2 thru_hole oval (at 0 2.54) (size 1.7 1.7) (drill 1) (layers *.Cu *.Mask) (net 5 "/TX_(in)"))
  (pad 1 thru_hole rect (at 0 0) (size 1.7 1.7) (drill 1) (layers *.Cu *.Mask) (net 4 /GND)))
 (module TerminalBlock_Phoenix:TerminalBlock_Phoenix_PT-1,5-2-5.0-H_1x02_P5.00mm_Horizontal (layer F.Cu) (at 169 112.5 270)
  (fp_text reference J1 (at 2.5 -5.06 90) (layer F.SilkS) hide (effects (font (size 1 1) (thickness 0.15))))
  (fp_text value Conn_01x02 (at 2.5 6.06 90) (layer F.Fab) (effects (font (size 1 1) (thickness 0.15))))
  (fp_line (start -2.8 5.3) (end -2.4 5.3) (layer F.SilkS) (width 0.12))
  (fp_line (start -2.8 4.66) (end -2.8 5.3) (layer F.SilkS) (width 0.12))
  (fp_line (start 3.742 0.992) (end 3.347 1.388) (layer F.SilkS) (width 0.12))
  (fp_line (start 6.388 -1.654) (end 6.008 -1.274) (layer F.SilkS) (width 0.12))
  (fp_line (start 3.993 1.274) (end 3.613 1.654) (layer F.SilkS) (width 0.12))
  (fp_line (start 6.654 -1.388) (end 6.259 -0.992) (layer F.SilkS) (width 0.12))
  (fp_line (start -1.548 1.281) (end -1.654 1.388) (layer F.SilkS) (width 0.12))
  (fp_line (start 1.388 -1.654) (end 1.281 -1.547) (layer F.SilkS) (width 0.12))
  (fp_line (start -1.282 1.547) (end -1.388 1.654) (layer F.SilkS) (width 0.12))
  (fp_line (start 1.654 -1.388) (end 1.547 -1.281) (layer F.SilkS) (width 0.12))
  (fp_line (start 7.56 -4.06) (end 7.56 5.06) (layer F.SilkS) (width 0.12))
  (fp_line (start -2.56 -4.06) (end -2.56 5.06) (layer F.SilkS) (width 0.12))
  (fp_line (start -2.56 5.06) (end 7.56 5.06) (layer F.SilkS) (width 0.12))
  (fp_line (start -2.56 -4.06) (end 7.56 -4.06) (layer F.SilkS) (width 0.12))
  (fp_line (start -2.56 3.5) (end 7.56 3.5) (layer F.SilkS) (width 0.12))
  (fp_line (start -2.56 4.6) (end 7.56 4.6) (layer F.SilkS) (width 0.12))
  (fp_circle (center 5 0) (end 7.18 0) (layer F.SilkS) (width 0.12))
  (fp_circle (center 0 0) (end 2.18 0) (layer F.SilkS) (width 0.12))
  (pad 2 thru_hole circle (at 5 0 270) (size 2.6 2.6) (drill 1.3) (layers *.Cu *.Mask) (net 2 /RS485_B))
  (pad 1 thru_hole rect (at 0 0 270) (size 2.6 2.6) (drill 1.3) (layers *.Cu *.Mask) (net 3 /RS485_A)))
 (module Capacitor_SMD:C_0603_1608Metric (layer F.Cu) (at 179.595 118.81 180)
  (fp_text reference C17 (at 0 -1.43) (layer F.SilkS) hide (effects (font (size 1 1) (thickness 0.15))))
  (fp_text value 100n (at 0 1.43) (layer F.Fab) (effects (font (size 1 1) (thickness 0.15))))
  (fp_line (start -0.162779 0.51) (end 0.162779 0.51) (layer F.SilkS) (width 0.12))
  (fp_line (start -0.162779 -0.51) (end 0.162779 -0.51) (layer F.SilkS) (width 0.12))
  (pad 2 smd roundrect (at 0.7875 0 180) (size 0.875 0.95) (layers F.Cu F.Paste F.Mask) (roundrect_rratio 0.25) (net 1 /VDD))
  (pad 1 smd roundrect (at -0.7875 0 180) (size 0.875 0.95) (layers F.Cu F.Paste F.Mask) (roundrect_rratio 0.25) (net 4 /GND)))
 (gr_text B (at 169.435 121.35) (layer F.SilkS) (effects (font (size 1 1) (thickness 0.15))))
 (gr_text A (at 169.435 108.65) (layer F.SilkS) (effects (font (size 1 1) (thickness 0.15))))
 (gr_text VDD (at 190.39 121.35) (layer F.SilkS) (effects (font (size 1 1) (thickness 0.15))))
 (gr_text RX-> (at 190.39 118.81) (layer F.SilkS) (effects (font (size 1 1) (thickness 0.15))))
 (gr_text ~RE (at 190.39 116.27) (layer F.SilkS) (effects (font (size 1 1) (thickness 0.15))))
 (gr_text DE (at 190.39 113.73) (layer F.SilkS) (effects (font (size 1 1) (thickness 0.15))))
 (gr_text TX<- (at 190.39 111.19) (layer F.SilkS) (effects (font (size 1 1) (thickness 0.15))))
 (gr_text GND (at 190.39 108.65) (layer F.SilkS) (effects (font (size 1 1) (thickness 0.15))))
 (gr_line (start 205.5 106) (end 181.5 106) (layer Edge.Cuts) (width 0.05))
 (gr_line (start 205.5 124) (end 205.5 106) (layer Edge.Cuts) (width 0.05))
 (gr_line (start 163.5 124) (end 205.5 124) (layer Edge.Cuts) (width 0.05))
 (gr_line (start 163.5 106) (end 163.5 124) (layer Edge.Cuts) (width 0.05))
 (gr_line (start 181.5 106) (end 163.5 106) (layer Edge.Cuts) (width 0.05))
 (segment (start 178.8075 117.1225) (end 179.025 116.905) (width 0.25) (layer F.Cu) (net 1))
 (segment (start 178.8075 118.81) (end 178.8075 117.1225) (width 0.25) (layer F.Cu) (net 1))
 (segment (start 178.8075 120.6075) (end 178.8075 118.81) (width 0.25) (layer F.Cu) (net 1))
 (segment (start 194.2 121.35) (end 179.55 121.35) (width 0.25) (layer F.Cu) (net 1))
 (segment (start 179.55 121.35) (end 178.8075 120.6075) (width 0.25) (layer F.Cu) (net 1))
 (segment (start 175.2125 117.5) (end 175.5 117.7875) (width 0.25) (layer F.Cu) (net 2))
 (segment (start 169 117.5) (end 175.2125 117.5) (width 0.25) (layer F.Cu) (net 2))
 (segment (start 175.5 117.7875) (end 176.8125 117.7875) (width 0.25) (layer F.Cu) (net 2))
 (segment (start 176.8125 117.7875) (end 177.2 117.4) (width 0.25) (layer F.Cu) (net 2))
 (segment (start 177.2 117.4) (end 177.2 116.1) (width 0.25) (layer F.Cu) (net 2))
 (segment (start 177.665 115.635) (end 179.025 115.635) (width 0.25) (layer F.Cu) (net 2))
 (segment (start 177.2 116.1) (end 177.665 115.635) (width 0.25) (layer F.Cu) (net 2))
 (segment (start 175.35 112.5) (end 175.5 112.35) (width 0.25) (layer F.Cu) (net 3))
 (segment (start 169 112.5) (end 175.35 112.5) (width 0.25) (layer F.Cu) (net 3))
 (segment (start 175.5 112.35) (end 176.75 112.35) (width 0.25) (layer F.Cu) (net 3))
 (segment (start 176.75 112.35) (end 177.2 112.8) (width 0.25) (layer F.Cu) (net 3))
 (segment (start 177.2 112.8) (end 177.2 113.9) (width 0.25) (layer F.Cu) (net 3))
 (segment (start 177.665 114.365) (end 179.025 114.365) (width 0.25) (layer F.Cu) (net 3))
 (segment (start 177.2 113.9) (end 177.665 114.365) (width 0.25) (layer F.Cu) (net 3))
 (segment (start 186.985 114.365) (end 187 114.35) (width 0.25) (layer F.Cu) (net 6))
 (segment (start 183.975 114.365) (end 186.985 114.365) (width 0.25) (layer F.Cu) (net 6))
 (segment (start 187 114.35) (end 188.55 114.35) (width 0.25) (layer F.Cu) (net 6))
 (segment (start 189.17 113.73) (end 191.025 113.73) (width 0.25) (layer F.Cu) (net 6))
 (segment (start 188.55 114.35) (end 189.17 113.73) (width 0.25) (layer F.Cu) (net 6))
 (segment (start 191.025 113.73) (end 194.2 113.73) (width 0.25) (layer F.Cu) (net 6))
 (segment (start 186.985 115.635) (end 187 115.65) (width 0.25) (layer F.Cu) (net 7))
 (segment (start 183.975 115.635) (end 186.985 115.635) (width 0.25) (layer F.Cu) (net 7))
 (segment (start 187 115.65) (end 188.55 115.65) (width 0.25) (layer F.Cu) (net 7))
 (segment (start 189.17 116.27) (end 191.025 116.27) (width 0.25) (layer F.Cu) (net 7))
 (segment (start 188.55 115.65) (end 189.17 116.27) (width 0.25) (layer F.Cu) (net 7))
 (segment (start 191.025 116.27) (end 194.2 116.27) (width 0.25) (layer F.Cu) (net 7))
 (segment (start 183.975 116.905) (end 185.605 116.905) (width 0.25) (layer F.Cu) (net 8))
 (segment (start 187.51 118.81) (end 191.025 118.81) (width 0.25) (layer F.Cu) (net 8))
 (segment (start 185.605 116.905) (end 187.51 118.81) (width 0.25) (layer F.Cu) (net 8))
 (segment (start 191.025 118.81) (end 194.2 118.81) (width 0.25) (layer F.Cu) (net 8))
 (segment (start 194.2 111.19) (end 187.61 111.19) (width 0.25) (layer F.Cu) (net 5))
 (segment (start 185.705 113.095) (end 183.975 113.095) (width 0.25) (layer F.Cu) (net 5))
 (segment (start 187.61 111.19) (end 185.705 113.095) (width 0.25) (layer F.Cu) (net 5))
 (segment (start 175.5 113.65) (end 175.5 116.2125) (width 0.25) (layer F.Cu) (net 9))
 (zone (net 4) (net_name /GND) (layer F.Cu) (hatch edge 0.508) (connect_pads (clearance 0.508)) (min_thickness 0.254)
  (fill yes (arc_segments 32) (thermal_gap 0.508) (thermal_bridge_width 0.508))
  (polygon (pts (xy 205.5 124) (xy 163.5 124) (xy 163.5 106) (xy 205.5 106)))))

